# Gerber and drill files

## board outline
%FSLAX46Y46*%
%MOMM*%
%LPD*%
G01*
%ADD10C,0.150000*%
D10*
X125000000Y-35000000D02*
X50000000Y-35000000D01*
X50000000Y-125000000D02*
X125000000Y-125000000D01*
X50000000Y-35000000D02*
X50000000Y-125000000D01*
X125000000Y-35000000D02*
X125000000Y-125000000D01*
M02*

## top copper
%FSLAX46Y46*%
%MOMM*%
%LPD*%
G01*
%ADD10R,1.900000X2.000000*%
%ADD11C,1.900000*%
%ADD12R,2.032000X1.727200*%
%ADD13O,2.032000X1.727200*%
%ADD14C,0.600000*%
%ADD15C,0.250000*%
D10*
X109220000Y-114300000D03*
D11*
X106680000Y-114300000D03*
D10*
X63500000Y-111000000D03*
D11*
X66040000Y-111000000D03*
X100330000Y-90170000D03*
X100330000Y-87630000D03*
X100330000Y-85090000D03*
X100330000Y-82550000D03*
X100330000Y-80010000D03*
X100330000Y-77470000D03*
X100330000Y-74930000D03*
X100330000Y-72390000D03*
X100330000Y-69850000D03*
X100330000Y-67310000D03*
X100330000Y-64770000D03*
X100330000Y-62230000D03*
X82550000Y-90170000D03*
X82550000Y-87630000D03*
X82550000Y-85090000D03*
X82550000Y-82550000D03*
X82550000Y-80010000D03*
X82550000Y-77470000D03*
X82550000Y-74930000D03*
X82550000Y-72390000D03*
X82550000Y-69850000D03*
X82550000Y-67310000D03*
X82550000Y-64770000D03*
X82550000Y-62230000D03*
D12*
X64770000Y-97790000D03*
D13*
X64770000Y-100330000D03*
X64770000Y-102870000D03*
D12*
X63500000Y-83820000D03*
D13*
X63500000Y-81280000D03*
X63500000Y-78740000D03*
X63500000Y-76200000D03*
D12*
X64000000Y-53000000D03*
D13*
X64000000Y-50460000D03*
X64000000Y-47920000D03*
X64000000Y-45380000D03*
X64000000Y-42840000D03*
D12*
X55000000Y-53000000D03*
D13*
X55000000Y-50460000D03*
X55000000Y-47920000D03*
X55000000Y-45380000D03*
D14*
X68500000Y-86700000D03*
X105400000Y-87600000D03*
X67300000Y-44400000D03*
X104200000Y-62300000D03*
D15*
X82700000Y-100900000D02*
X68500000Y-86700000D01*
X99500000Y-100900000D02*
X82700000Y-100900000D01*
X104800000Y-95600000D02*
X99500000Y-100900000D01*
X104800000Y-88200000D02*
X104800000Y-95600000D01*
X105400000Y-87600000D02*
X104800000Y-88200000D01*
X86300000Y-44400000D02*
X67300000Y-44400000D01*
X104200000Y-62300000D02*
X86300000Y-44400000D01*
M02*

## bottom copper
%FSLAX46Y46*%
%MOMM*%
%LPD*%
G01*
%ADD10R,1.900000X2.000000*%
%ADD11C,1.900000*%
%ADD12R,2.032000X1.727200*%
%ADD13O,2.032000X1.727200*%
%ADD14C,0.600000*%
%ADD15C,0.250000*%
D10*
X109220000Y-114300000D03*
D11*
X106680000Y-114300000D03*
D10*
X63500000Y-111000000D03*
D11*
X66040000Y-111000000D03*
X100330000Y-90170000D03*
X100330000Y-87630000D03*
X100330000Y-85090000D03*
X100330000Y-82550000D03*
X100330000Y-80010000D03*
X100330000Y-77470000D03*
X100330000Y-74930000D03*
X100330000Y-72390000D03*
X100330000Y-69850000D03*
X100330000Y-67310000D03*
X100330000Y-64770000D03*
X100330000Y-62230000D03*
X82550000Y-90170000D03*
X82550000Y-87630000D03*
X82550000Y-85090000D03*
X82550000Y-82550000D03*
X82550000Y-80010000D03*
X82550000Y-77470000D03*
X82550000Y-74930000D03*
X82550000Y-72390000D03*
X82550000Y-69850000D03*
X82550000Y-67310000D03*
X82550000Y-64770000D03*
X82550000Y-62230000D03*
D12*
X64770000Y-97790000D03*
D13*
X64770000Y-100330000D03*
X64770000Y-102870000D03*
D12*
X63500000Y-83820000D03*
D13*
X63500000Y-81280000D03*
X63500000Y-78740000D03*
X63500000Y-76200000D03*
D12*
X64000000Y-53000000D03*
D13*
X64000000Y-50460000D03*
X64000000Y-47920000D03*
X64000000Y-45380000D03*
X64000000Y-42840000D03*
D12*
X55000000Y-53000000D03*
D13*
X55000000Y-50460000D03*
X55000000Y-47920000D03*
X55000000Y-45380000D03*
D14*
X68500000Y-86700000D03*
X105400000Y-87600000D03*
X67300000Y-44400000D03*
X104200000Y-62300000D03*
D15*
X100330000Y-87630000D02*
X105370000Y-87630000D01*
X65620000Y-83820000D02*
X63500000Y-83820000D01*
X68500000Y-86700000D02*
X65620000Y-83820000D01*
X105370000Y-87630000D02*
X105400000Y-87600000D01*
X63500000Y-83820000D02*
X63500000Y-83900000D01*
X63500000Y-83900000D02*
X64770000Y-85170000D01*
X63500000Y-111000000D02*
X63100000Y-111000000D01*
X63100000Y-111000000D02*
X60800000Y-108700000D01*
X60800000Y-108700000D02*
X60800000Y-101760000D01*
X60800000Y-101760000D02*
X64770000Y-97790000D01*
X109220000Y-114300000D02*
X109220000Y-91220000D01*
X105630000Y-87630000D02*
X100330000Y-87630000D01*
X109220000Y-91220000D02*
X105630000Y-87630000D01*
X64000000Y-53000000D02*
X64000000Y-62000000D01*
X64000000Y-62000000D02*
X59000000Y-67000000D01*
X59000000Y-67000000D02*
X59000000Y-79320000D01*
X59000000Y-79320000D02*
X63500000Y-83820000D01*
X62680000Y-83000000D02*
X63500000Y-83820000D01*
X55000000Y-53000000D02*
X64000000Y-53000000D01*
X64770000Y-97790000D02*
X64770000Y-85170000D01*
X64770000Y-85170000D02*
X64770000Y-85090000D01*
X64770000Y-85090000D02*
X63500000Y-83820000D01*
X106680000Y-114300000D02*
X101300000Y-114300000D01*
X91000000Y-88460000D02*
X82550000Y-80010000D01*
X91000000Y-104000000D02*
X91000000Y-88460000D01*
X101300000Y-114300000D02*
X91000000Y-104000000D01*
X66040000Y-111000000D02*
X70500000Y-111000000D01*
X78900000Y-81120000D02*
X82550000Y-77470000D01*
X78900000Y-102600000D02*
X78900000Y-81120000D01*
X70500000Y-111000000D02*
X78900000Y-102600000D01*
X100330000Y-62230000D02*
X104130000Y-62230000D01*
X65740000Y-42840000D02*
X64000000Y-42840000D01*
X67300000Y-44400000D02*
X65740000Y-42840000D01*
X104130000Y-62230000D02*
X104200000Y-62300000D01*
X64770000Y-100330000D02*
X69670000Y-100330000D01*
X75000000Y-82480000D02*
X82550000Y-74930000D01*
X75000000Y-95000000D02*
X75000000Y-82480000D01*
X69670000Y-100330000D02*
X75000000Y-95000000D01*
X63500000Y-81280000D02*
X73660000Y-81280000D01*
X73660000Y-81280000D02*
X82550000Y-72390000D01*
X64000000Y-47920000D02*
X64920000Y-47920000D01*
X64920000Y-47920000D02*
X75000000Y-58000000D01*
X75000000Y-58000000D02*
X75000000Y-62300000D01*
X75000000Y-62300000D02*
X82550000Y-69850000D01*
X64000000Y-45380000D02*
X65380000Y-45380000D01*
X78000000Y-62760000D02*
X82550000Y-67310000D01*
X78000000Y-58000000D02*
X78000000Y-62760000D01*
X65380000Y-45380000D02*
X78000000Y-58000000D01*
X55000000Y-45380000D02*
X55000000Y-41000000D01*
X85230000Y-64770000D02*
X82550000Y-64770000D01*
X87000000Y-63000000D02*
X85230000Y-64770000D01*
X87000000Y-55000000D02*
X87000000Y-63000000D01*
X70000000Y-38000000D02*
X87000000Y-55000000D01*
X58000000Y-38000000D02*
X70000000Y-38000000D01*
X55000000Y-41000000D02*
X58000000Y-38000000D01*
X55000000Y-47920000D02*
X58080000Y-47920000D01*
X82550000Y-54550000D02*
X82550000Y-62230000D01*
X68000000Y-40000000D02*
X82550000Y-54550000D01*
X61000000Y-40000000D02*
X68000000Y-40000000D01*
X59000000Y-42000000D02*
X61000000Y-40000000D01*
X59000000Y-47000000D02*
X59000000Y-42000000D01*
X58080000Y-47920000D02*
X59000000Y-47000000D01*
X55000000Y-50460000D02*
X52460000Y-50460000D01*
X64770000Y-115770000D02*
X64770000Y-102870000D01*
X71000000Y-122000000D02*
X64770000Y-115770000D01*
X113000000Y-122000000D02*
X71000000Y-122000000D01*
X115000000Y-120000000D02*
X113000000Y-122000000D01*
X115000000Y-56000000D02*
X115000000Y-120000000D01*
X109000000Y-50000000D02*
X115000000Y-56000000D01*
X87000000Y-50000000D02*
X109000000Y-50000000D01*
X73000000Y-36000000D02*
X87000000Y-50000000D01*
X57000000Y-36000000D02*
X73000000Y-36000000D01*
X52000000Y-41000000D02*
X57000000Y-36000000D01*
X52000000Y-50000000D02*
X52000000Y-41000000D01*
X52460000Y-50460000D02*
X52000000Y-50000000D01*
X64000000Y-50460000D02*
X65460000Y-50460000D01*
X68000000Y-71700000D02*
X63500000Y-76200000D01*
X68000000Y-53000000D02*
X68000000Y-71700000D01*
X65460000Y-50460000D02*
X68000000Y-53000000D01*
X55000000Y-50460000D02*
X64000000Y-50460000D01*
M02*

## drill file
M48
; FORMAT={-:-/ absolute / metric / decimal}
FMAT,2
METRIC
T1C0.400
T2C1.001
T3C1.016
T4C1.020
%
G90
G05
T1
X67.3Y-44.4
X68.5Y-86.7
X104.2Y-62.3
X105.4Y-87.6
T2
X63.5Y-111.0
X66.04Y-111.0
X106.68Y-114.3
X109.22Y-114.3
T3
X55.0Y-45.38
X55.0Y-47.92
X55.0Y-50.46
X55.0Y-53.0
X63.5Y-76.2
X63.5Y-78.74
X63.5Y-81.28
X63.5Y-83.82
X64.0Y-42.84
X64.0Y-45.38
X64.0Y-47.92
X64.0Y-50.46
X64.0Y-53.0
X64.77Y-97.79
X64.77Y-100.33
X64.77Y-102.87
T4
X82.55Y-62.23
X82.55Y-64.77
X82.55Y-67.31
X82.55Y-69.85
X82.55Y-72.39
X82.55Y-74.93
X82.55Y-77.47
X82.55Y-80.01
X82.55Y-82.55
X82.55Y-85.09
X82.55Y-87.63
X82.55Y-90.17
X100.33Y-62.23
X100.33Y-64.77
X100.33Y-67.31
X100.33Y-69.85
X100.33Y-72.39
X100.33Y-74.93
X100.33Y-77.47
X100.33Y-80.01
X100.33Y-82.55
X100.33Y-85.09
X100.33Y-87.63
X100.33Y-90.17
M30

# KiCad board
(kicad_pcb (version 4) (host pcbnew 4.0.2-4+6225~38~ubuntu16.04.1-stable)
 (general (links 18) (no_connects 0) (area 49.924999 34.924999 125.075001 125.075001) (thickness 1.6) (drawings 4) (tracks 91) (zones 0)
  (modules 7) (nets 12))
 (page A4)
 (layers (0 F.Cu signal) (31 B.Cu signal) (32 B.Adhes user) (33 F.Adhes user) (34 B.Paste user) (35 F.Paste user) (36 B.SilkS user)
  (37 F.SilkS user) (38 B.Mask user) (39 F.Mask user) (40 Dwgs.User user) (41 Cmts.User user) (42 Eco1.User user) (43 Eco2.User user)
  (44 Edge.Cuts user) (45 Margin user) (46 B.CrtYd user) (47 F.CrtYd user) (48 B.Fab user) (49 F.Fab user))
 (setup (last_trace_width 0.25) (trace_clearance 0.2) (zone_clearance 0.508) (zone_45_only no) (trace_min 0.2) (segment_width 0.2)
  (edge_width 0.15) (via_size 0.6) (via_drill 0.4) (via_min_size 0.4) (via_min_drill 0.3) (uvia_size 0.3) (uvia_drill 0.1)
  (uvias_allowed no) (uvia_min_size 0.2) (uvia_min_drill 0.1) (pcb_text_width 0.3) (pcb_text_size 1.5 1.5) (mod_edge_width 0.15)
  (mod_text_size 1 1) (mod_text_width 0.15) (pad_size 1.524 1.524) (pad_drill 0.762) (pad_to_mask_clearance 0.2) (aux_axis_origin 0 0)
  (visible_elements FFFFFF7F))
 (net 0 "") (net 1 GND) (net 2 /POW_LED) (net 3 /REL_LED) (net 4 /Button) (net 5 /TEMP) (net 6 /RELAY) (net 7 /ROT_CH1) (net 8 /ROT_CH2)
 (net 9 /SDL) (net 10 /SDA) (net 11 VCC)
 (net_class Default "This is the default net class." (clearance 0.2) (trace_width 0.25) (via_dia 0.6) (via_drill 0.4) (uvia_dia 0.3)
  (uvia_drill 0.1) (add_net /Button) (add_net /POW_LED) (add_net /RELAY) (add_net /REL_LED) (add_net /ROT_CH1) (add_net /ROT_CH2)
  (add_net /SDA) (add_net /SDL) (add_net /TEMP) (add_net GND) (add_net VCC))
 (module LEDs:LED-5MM (layer F.Cu) (at 109.22 114.3 180)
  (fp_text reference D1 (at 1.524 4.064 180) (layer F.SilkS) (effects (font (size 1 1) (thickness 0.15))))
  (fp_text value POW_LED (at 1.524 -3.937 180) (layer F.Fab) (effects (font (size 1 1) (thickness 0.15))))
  (pad 1 thru_hole rect (at 0 0 270) (size 2 1.9) (drill 1.00076) (layers *.Cu *.Mask F.SilkS) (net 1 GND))
  (pad 2 thru_hole circle (at 2.54 0 180) (size 1.9 1.9) (drill 1.00076) (layers *.Cu *.Mask F.SilkS) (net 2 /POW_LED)))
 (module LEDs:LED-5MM (layer F.Cu) (at 63.5 111)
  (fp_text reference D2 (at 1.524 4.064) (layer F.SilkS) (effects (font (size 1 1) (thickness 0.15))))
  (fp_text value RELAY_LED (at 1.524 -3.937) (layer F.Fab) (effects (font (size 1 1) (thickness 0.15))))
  (pad 1 thru_hole rect (at 0 0 90) (size 2 1.9) (drill 1.00076) (layers *.Cu *.Mask F.SilkS) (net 1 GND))
  (pad 2 thru_hole circle (at 2.54 0) (size 1.9 1.9) (drill 1.00076) (layers *.Cu *.Mask F.SilkS) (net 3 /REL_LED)))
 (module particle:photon (layer F.Cu) (at 91.44 74.93 180)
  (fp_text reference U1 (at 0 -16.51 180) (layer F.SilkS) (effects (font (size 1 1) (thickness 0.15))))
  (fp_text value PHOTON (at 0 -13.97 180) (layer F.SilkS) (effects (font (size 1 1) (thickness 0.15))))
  (pad 1 thru_hole circle (at -8.89 -15.24 180) (size 1.9 1.9) (drill 1.02) (layers *.Cu *.Mask F.SilkS))
  (pad 2 thru_hole circle (at -8.89 -12.7 180) (size 1.9 1.9) (drill 1.02) (layers *.Cu *.Mask F.SilkS) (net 1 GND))
  (pad 3 thru_hole circle (at -8.89 -10.16 180) (size 1.9 1.9) (drill 1.02) (layers *.Cu *.Mask F.SilkS))
  (pad 4 thru_hole circle (at -8.89 -7.62 180) (size 1.9 1.9) (drill 1.02) (layers *.Cu *.Mask F.SilkS))
  (pad 5 thru_hole circle (at -8.89 -5.08 180) (size 1.9 1.9) (drill 1.02) (layers *.Cu *.Mask F.SilkS))
  (pad 6 thru_hole circle (at -8.89 -2.54 180) (size 1.9 1.9) (drill 1.02) (layers *.Cu *.Mask F.SilkS))
  (pad 7 thru_hole circle (at -8.89 0 180) (size 1.9 1.9) (drill 1.02) (layers *.Cu *.Mask F.SilkS))
  (pad 8 thru_hole circle (at -8.89 2.54 180) (size 1.9 1.9) (drill 1.02) (layers *.Cu *.Mask F.SilkS))
  (pad 9 thru_hole circle (at -8.89 5.08 180) (size 1.9 1.9) (drill 1.02) (layers *.Cu *.Mask F.SilkS))
  (pad 10 thru_hole circle (at -8.89 7.62 180) (size 1.9 1.9) (drill 1.02) (layers *.Cu *.Mask F.SilkS))
  (pad 11 thru_hole circle (at -8.89 10.16 180) (size 1.9 1.9) (drill 1.02) (layers *.Cu *.Mask F.SilkS))
  (pad 12 thru_hole circle (at -8.89 12.7 180) (size 1.9 1.9) (drill 1.02) (layers *.Cu *.Mask F.SilkS) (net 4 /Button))
  (pad 24 thru_hole circle (at 8.89 -15.24 180) (size 1.9 1.9) (drill 1.02) (layers *.Cu *.Mask F.SilkS))
  (pad 23 thru_hole circle (at 8.89 -12.7 180) (size 1.9 1.9) (drill 1.02) (layers *.Cu *.Mask F.SilkS))
  (pad 22 thru_hole circle (at 8.89 -10.16 180) (size 1.9 1.9) (drill 1.02) (layers *.Cu *.Mask F.SilkS))
  (pad 21 thru_hole circle (at 8.89 -7.62 180) (size 1.9 1.9) (drill 1.02) (layers *.Cu *.Mask F.SilkS))
  (pad 20 thru_hole circle (at 8.89 -5.08 180) (size 1.9 1.9) (drill 1.02) (layers *.Cu *.Mask F.SilkS) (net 2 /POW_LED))
  (pad 19 thru_hole circle (at 8.89 -2.54 180) (size 1.9 1.9) (drill 1.02) (layers *.Cu *.Mask F.SilkS) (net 3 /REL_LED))
  (pad 18 thru_hole circle (at 8.89 0 180) (size 1.9 1.9) (drill 1.02) (layers *.Cu *.Mask F.SilkS) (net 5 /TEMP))
  (pad 17 thru_hole circle (at 8.89 2.54 180) (size 1.9 1.9) (drill 1.02) (layers *.Cu *.Mask F.SilkS) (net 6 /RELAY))
  (pad 16 thru_hole circle (at 8.89 5.08 180) (size 1.9 1.9) (drill 1.02) (layers *.Cu *.Mask F.SilkS) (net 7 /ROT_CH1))
  (pad 15 thru_hole circle (at 8.89 7.62 180) (size 1.9 1.9) (drill 1.02) (layers *.Cu *.Mask F.SilkS) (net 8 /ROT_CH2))
  (pad 14 thru_hole circle (at 8.89 10.16 180) (size 1.9 1.9) (drill 1.02) (layers *.Cu *.Mask F.SilkS) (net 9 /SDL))
  (pad 13 thru_hole circle (at 8.89 12.7 180) (size 1.9 1.9) (drill 1.02) (layers *.Cu *.Mask F.SilkS) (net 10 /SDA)))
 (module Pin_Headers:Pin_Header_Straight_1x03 (layer F.Cu) (at 64.77 97.79)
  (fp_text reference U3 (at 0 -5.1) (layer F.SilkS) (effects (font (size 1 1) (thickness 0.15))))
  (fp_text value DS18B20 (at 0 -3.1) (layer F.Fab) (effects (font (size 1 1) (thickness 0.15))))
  (pad 1 thru_hole rect (at 0 0) (size 2.032 1.7272) (drill 1.016) (layers *.Cu *.Mask F.SilkS) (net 1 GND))
  (pad 2 thru_hole oval (at 0 2.54) (size 2.032 1.7272) (drill 1.016) (layers *.Cu *.Mask F.SilkS) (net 5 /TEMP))
  (pad 3 thru_hole oval (at 0 5.08) (size 2.032 1.7272) (drill 1.016) (layers *.Cu *.Mask F.SilkS) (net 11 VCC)))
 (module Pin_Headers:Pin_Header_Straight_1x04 (layer F.Cu) (at 63.5 83.82 180)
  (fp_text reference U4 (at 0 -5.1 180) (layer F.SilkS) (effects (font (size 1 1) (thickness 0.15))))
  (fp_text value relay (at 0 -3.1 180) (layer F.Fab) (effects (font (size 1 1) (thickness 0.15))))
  (pad 1 thru_hole rect (at 0 0 180) (size 2.032 1.7272) (drill 1.016) (layers *.Cu *.Mask F.SilkS) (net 1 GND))
  (pad 2 thru_hole oval (at 0 2.54 180) (size 2.032 1.7272) (drill 1.016) (layers *.Cu *.Mask F.SilkS) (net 6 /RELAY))
  (pad 3 thru_hole oval (at 0 5.08 180) (size 2.032 1.7272) (drill 1.016) (layers *.Cu *.Mask F.SilkS))
  (pad 4 thru_hole oval (at 0 7.62 180) (size 2.032 1.7272) (drill 1.016) (layers *.Cu *.Mask F.SilkS) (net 11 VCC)))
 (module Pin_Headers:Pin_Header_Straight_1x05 (layer F.Cu) (at 64 53 180)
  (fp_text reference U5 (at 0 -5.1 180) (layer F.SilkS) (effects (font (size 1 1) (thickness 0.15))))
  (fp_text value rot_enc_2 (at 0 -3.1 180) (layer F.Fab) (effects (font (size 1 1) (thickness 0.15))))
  (pad 1 thru_hole rect (at 0 0 180) (size 2.032 1.7272) (drill 1.016) (layers *.Cu *.Mask F.SilkS) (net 1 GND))
  (pad 2 thru_hole oval (at 0 2.54 180) (size 2.032 1.7272) (drill 1.016) (layers *.Cu *.Mask F.SilkS) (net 11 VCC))
  (pad 3 thru_hole oval (at 0 5.08 180) (size 2.032 1.7272) (drill 1.016) (layers *.Cu *.Mask F.SilkS) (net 7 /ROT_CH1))
  (pad 4 thru_hole oval (at 0 7.62 180) (size 2.032 1.7272) (drill 1.016) (layers *.Cu *.Mask F.SilkS) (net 8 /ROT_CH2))
  (pad 5 thru_hole oval (at 0 10.16 180) (size 2.032 1.7272) (drill 1.016) (layers *.Cu *.Mask F.SilkS) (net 4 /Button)))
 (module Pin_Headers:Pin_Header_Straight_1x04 (layer F.Cu) (at 55 53 180)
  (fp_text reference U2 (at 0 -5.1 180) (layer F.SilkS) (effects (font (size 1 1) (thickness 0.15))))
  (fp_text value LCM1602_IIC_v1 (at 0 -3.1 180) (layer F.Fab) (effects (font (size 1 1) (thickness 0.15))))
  (pad 1 thru_hole rect (at 0 0 180) (size 2.032 1.7272) (drill 1.016) (layers *.Cu *.Mask F.SilkS) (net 1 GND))
  (pad 2 thru_hole oval (at 0 2.54 180) (size 2.032 1.7272) (drill 1.016) (layers *.Cu *.Mask F.SilkS) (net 11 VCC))
  (pad 3 thru_hole oval (at 0 5.08 180) (size 2.032 1.7272) (drill 1.016) (layers *.Cu *.Mask F.SilkS) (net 10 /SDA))
  (pad 4 thru_hole oval (at 0 7.62 180) (size 2.032 1.7272) (drill 1.016) (layers *.Cu *.Mask F.SilkS) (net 9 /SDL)))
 (gr_line (start 125 35) (end 50 35) (angle 90) (layer Edge.Cuts) (width 0.15))
 (gr_line (start 50 125) (end 125 125) (angle 90) (layer Edge.Cuts) (width 0.15))
 (gr_line (start 50 35) (end 50 125) (angle 90) (layer Edge.Cuts) (width 0.15))
 (gr_line (start 125 35) (end 125 125) (angle 90) (layer Edge.Cuts) (width 0.15))
 (segment (start 100.33 87.63) (end 105.37 87.63) (width 0.25) (layer B.Cu) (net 1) (status 400000))
 (segment (start 65.62 83.82) (end 63.5 83.82) (width 0.25) (layer B.Cu) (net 1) (status 800000))
 (segment (start 68.5 86.7) (end 65.62 83.82) (width 0.25) (layer B.Cu) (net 1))
 (via (at 68.5 86.7) (size 0.6) (drill 0.4) (layers F.Cu B.Cu) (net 1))
 (segment (start 82.7 100.9) (end 68.5 86.7) (width 0.25) (layer F.Cu) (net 1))
 (segment (start 99.5 100.9) (end 82.7 100.9) (width 0.25) (layer F.Cu) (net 1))
 (segment (start 104.8 95.6) (end 99.5 100.9) (width 0.25) (layer F.Cu) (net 1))
 (segment (start 104.8 88.2) (end 104.8 95.6) (width 0.25) (layer F.Cu) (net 1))
 (segment (start 105.4 87.6) (end 104.8 88.2) (width 0.25) (layer F.Cu) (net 1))
 (via (at 105.4 87.6) (size 0.6) (drill 0.4) (layers F.Cu B.Cu) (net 1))
 (segment (start 105.37 87.63) (end 105.4 87.6) (width 0.25) (layer B.Cu) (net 1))
 (segment (start 63.5 83.82) (end 63.5 83.9) (width 0.25) (layer B.Cu) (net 1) (status C00000))
 (segment (start 63.5 83.9) (end 64.77 85.17) (width 0.25) (layer B.Cu) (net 1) (status 400000))
 (segment (start 63.5 111) (end 63.1 111) (width 0.25) (layer B.Cu) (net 1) (status C00000))
 (segment (start 63.1 111) (end 60.8 108.7) (width 0.25) (layer B.Cu) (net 1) (status 400000))
 (segment (start 60.8 108.7) (end 60.8 101.76) (width 0.25) (layer B.Cu) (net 1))
 (segment (start 60.8 101.76) (end 64.77 97.79) (width 0.25) (layer B.Cu) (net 1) (status 800000))
 (segment (start 109.22 114.3) (end 109.22 91.22) (width 0.25) (layer B.Cu) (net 1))
 (segment (start 105.63 87.63) (end 100.33 87.63) (width 0.25) (layer B.Cu) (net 1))
 (segment (start 109.22 91.22) (end 105.63 87.63) (width 0.25) (layer B.Cu) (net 1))
 (segment (start 64 53) (end 64 62) (width 0.25) (layer B.Cu) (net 1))
 (segment (start 64 62) (end 59 67) (width 0.25) (layer B.Cu) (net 1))
 (segment (start 59 67) (end 59 79.32) (width 0.25) (layer B.Cu) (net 1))
 (segment (start 59 79.32) (end 63.5 83.82) (width 0.25) (layer B.Cu) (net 1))
 (segment (start 62.68 83) (end 63.5 83.82) (width 0.25) (layer B.Cu) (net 1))
 (segment (start 55 53) (end 64 53) (width 0.25) (layer B.Cu) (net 1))
 (segment (start 64.77 97.79) (end 64.77 85.17) (width 0.25) (layer B.Cu) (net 1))
 (segment (start 64.77 85.17) (end 64.77 85.09) (width 0.25) (layer B.Cu) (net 1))
 (segment (start 64.77 85.09) (end 63.5 83.82) (width 0.25) (layer B.Cu) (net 1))
 (segment (start 106.68 114.3) (end 101.3 114.3) (width 0.25) (layer B.Cu) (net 2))
 (segment (start 91 88.46) (end 82.55 80.01) (width 0.25) (layer B.Cu) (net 2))
 (segment (start 91 104) (end 91 88.46) (width 0.25) (layer B.Cu) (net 2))
 (segment (start 101.3 114.3) (end 91 104) (width 0.25) (layer B.Cu) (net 2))
 (segment (start 66.04 111) (end 70.5 111) (width 0.25) (layer B.Cu) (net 3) (status 400000))
 (segment (start 78.9 81.12) (end 82.55 77.47) (width 0.25) (layer B.Cu) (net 3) (status 800000))
 (segment (start 78.9 102.6) (end 78.9 81.12) (width 0.25) (layer B.Cu) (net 3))
 (segment (start 70.5 111) (end 78.9 102.6) (width 0.25) (layer B.Cu) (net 3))
 (segment (start 100.33 62.23) (end 104.13 62.23) (width 0.25) (layer B.Cu) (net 4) (status 400000))
 (segment (start 65.74 42.84) (end 64 42.84) (width 0.25) (layer B.Cu) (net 4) (status 800000))
 (segment (start 67.3 44.4) (end 65.74 42.84) (width 0.25) (layer B.Cu) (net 4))
 (via (at 67.3 44.4) (size 0.6) (drill 0.4) (layers F.Cu B.Cu) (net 4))
 (segment (start 86.3 44.4) (end 67.3 44.4) (width 0.25) (layer F.Cu) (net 4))
 (segment (start 104.2 62.3) (end 86.3 44.4) (width 0.25) (layer F.Cu) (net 4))
 (via (at 104.2 62.3) (size 0.6) (drill 0.4) (layers F.Cu B.Cu) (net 4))
 (segment (start 104.13 62.23) (end 104.2 62.3) (width 0.25) (layer B.Cu) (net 4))
 (segment (start 64.77 100.33) (end 69.67 100.33) (width 0.25) (layer B.Cu) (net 5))
 (segment (start 75 82.48) (end 82.55 74.93) (width 0.25) (layer B.Cu) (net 5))
 (segment (start 75 95) (end 75 82.48) (width 0.25) (layer B.Cu) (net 5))
 (segment (start 69.67 100.33) (end 75 95) (width 0.25) (layer B.Cu) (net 5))
 (segment (start 63.5 81.28) (end 73.66 81.28) (width 0.25) (layer B.Cu) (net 6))
 (segment (start 73.66 81.28) (end 82.55 72.39) (width 0.25) (layer B.Cu) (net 6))
 (segment (start 64 47.92) (end 64.92 47.92) (width 0.25) (layer B.Cu) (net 7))
 (segment (start 64.92 47.92) (end 75 58) (width 0.25) (layer B.Cu) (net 7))
 (segment (start 75 58) (end 75 62.3) (width 0.25) (layer B.Cu) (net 7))
 (segment (start 75 62.3) (end 82.55 69.85) (width 0.25) (layer B.Cu) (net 7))
 (segment (start 64 45.38) (end 65.38 45.38) (width 0.25) (layer B.Cu) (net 8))
 (segment (start 78 62.76) (end 82.55 67.31) (width 0.25) (layer B.Cu) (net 8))
 (segment (start 78 58) (end 78 62.76) (width 0.25) (layer B.Cu) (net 8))
 (segment (start 65.38 45.38) (end 78 58) (width 0.25) (layer B.Cu) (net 8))
 (segment (start 55 45.38) (end 55 41) (width 0.25) (layer B.Cu) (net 9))
 (segment (start 85.23 64.77) (end 82.55 64.77) (width 0.25) (layer B.Cu) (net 9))
 (segment (start 87 63) (end 85.23 64.77) (width 0.25) (layer B.Cu) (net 9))
 (segment (start 87 55) (end 87 63) (width 0.25) (layer B.Cu) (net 9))
 (segment (start 70 38) (end 87 55) (width 0.25) (layer B.Cu) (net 9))
 (segment (start 58 38) (end 70 38) (width 0.25) (layer B.Cu) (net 9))
 (segment (start 55 41) (end 58 38) (width 0.25) (layer B.Cu) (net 9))
 (segment (start 55 47.92) (end 58.08 47.92) (width 0.25) (layer B.Cu) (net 10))
 (segment (start 82.55 54.55) (end 82.55 62.23) (width 0.25) (layer B.Cu) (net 10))
 (segment (start 68 40) (end 82.55 54.55) (width 0.25) (layer B.Cu) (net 10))
 (segment (start 61 40) (end 68 40) (width 0.25) (layer B.Cu) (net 10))
 (segment (start 59 42) (end 61 40) (width 0.25) (layer B.Cu) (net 10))
 (segment (start 59 47) (end 59 42) (width 0.25) (layer B.Cu) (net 10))
 (segment (start 58.08 47.92) (end 59 47) (width 0.25) (layer B.Cu) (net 10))
 (segment (start 55 50.46) (end 52.46 50.46) (width 0.25) (layer B.Cu) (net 11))
 (segment (start 64.77 115.77) (end 64.77 102.87) (width 0.25) (layer B.Cu) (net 11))
 (segment (start 71 122) (end 64.77 115.77) (width 0.25) (layer B.Cu) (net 11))
 (segment (start 113 122) (end 71 122) (width 0.25) (layer B.Cu) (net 11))
 (segment (start 115 120) (end 113 122) (width 0.25) (layer B.Cu) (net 11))
 (segment (start 115 56) (end 115 120) (width 0.25) (layer B.Cu) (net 11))
 (segment (start 109 50) (end 115 56) (width 0.25) (layer B.Cu) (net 11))
 (segment (start 87 50) (end 109 50) (width 0.25) (layer B.Cu) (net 11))
 (segment (start 73 36) (end 87 50) (width 0.25) (layer B.Cu) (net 11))
 (segment (start 57 36) (end 73 36) (width 0.25) (layer B.Cu) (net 11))
 (segment (start 52 41) (end 57 36) (width 0.25) (layer B.Cu) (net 11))
 (segment (start 52 50) (end 52 41) (width 0.25) (layer B.Cu) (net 11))
 (segment (start 52.46 50.46) (end 52 50) (width 0.25) (layer B.Cu) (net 11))
 (segment (start 64 50.46) (end 65.46 50.46) (width 0.25) (layer B.Cu) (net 11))
 (segment (start 68 71.7) (end 63.5 76.2) (width 0.25) (layer B.Cu) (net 11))
 (segment (start 68 53) (end 68 71.7) (width 0.25) (layer B.Cu) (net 11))
 (segment (start 65.46 50.46) (end 68 53) (width 0.25) (layer B.Cu) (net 11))
 (segment (start 55 50.46) (end 64 50.46) (width 0.25) (layer B.Cu) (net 11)))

